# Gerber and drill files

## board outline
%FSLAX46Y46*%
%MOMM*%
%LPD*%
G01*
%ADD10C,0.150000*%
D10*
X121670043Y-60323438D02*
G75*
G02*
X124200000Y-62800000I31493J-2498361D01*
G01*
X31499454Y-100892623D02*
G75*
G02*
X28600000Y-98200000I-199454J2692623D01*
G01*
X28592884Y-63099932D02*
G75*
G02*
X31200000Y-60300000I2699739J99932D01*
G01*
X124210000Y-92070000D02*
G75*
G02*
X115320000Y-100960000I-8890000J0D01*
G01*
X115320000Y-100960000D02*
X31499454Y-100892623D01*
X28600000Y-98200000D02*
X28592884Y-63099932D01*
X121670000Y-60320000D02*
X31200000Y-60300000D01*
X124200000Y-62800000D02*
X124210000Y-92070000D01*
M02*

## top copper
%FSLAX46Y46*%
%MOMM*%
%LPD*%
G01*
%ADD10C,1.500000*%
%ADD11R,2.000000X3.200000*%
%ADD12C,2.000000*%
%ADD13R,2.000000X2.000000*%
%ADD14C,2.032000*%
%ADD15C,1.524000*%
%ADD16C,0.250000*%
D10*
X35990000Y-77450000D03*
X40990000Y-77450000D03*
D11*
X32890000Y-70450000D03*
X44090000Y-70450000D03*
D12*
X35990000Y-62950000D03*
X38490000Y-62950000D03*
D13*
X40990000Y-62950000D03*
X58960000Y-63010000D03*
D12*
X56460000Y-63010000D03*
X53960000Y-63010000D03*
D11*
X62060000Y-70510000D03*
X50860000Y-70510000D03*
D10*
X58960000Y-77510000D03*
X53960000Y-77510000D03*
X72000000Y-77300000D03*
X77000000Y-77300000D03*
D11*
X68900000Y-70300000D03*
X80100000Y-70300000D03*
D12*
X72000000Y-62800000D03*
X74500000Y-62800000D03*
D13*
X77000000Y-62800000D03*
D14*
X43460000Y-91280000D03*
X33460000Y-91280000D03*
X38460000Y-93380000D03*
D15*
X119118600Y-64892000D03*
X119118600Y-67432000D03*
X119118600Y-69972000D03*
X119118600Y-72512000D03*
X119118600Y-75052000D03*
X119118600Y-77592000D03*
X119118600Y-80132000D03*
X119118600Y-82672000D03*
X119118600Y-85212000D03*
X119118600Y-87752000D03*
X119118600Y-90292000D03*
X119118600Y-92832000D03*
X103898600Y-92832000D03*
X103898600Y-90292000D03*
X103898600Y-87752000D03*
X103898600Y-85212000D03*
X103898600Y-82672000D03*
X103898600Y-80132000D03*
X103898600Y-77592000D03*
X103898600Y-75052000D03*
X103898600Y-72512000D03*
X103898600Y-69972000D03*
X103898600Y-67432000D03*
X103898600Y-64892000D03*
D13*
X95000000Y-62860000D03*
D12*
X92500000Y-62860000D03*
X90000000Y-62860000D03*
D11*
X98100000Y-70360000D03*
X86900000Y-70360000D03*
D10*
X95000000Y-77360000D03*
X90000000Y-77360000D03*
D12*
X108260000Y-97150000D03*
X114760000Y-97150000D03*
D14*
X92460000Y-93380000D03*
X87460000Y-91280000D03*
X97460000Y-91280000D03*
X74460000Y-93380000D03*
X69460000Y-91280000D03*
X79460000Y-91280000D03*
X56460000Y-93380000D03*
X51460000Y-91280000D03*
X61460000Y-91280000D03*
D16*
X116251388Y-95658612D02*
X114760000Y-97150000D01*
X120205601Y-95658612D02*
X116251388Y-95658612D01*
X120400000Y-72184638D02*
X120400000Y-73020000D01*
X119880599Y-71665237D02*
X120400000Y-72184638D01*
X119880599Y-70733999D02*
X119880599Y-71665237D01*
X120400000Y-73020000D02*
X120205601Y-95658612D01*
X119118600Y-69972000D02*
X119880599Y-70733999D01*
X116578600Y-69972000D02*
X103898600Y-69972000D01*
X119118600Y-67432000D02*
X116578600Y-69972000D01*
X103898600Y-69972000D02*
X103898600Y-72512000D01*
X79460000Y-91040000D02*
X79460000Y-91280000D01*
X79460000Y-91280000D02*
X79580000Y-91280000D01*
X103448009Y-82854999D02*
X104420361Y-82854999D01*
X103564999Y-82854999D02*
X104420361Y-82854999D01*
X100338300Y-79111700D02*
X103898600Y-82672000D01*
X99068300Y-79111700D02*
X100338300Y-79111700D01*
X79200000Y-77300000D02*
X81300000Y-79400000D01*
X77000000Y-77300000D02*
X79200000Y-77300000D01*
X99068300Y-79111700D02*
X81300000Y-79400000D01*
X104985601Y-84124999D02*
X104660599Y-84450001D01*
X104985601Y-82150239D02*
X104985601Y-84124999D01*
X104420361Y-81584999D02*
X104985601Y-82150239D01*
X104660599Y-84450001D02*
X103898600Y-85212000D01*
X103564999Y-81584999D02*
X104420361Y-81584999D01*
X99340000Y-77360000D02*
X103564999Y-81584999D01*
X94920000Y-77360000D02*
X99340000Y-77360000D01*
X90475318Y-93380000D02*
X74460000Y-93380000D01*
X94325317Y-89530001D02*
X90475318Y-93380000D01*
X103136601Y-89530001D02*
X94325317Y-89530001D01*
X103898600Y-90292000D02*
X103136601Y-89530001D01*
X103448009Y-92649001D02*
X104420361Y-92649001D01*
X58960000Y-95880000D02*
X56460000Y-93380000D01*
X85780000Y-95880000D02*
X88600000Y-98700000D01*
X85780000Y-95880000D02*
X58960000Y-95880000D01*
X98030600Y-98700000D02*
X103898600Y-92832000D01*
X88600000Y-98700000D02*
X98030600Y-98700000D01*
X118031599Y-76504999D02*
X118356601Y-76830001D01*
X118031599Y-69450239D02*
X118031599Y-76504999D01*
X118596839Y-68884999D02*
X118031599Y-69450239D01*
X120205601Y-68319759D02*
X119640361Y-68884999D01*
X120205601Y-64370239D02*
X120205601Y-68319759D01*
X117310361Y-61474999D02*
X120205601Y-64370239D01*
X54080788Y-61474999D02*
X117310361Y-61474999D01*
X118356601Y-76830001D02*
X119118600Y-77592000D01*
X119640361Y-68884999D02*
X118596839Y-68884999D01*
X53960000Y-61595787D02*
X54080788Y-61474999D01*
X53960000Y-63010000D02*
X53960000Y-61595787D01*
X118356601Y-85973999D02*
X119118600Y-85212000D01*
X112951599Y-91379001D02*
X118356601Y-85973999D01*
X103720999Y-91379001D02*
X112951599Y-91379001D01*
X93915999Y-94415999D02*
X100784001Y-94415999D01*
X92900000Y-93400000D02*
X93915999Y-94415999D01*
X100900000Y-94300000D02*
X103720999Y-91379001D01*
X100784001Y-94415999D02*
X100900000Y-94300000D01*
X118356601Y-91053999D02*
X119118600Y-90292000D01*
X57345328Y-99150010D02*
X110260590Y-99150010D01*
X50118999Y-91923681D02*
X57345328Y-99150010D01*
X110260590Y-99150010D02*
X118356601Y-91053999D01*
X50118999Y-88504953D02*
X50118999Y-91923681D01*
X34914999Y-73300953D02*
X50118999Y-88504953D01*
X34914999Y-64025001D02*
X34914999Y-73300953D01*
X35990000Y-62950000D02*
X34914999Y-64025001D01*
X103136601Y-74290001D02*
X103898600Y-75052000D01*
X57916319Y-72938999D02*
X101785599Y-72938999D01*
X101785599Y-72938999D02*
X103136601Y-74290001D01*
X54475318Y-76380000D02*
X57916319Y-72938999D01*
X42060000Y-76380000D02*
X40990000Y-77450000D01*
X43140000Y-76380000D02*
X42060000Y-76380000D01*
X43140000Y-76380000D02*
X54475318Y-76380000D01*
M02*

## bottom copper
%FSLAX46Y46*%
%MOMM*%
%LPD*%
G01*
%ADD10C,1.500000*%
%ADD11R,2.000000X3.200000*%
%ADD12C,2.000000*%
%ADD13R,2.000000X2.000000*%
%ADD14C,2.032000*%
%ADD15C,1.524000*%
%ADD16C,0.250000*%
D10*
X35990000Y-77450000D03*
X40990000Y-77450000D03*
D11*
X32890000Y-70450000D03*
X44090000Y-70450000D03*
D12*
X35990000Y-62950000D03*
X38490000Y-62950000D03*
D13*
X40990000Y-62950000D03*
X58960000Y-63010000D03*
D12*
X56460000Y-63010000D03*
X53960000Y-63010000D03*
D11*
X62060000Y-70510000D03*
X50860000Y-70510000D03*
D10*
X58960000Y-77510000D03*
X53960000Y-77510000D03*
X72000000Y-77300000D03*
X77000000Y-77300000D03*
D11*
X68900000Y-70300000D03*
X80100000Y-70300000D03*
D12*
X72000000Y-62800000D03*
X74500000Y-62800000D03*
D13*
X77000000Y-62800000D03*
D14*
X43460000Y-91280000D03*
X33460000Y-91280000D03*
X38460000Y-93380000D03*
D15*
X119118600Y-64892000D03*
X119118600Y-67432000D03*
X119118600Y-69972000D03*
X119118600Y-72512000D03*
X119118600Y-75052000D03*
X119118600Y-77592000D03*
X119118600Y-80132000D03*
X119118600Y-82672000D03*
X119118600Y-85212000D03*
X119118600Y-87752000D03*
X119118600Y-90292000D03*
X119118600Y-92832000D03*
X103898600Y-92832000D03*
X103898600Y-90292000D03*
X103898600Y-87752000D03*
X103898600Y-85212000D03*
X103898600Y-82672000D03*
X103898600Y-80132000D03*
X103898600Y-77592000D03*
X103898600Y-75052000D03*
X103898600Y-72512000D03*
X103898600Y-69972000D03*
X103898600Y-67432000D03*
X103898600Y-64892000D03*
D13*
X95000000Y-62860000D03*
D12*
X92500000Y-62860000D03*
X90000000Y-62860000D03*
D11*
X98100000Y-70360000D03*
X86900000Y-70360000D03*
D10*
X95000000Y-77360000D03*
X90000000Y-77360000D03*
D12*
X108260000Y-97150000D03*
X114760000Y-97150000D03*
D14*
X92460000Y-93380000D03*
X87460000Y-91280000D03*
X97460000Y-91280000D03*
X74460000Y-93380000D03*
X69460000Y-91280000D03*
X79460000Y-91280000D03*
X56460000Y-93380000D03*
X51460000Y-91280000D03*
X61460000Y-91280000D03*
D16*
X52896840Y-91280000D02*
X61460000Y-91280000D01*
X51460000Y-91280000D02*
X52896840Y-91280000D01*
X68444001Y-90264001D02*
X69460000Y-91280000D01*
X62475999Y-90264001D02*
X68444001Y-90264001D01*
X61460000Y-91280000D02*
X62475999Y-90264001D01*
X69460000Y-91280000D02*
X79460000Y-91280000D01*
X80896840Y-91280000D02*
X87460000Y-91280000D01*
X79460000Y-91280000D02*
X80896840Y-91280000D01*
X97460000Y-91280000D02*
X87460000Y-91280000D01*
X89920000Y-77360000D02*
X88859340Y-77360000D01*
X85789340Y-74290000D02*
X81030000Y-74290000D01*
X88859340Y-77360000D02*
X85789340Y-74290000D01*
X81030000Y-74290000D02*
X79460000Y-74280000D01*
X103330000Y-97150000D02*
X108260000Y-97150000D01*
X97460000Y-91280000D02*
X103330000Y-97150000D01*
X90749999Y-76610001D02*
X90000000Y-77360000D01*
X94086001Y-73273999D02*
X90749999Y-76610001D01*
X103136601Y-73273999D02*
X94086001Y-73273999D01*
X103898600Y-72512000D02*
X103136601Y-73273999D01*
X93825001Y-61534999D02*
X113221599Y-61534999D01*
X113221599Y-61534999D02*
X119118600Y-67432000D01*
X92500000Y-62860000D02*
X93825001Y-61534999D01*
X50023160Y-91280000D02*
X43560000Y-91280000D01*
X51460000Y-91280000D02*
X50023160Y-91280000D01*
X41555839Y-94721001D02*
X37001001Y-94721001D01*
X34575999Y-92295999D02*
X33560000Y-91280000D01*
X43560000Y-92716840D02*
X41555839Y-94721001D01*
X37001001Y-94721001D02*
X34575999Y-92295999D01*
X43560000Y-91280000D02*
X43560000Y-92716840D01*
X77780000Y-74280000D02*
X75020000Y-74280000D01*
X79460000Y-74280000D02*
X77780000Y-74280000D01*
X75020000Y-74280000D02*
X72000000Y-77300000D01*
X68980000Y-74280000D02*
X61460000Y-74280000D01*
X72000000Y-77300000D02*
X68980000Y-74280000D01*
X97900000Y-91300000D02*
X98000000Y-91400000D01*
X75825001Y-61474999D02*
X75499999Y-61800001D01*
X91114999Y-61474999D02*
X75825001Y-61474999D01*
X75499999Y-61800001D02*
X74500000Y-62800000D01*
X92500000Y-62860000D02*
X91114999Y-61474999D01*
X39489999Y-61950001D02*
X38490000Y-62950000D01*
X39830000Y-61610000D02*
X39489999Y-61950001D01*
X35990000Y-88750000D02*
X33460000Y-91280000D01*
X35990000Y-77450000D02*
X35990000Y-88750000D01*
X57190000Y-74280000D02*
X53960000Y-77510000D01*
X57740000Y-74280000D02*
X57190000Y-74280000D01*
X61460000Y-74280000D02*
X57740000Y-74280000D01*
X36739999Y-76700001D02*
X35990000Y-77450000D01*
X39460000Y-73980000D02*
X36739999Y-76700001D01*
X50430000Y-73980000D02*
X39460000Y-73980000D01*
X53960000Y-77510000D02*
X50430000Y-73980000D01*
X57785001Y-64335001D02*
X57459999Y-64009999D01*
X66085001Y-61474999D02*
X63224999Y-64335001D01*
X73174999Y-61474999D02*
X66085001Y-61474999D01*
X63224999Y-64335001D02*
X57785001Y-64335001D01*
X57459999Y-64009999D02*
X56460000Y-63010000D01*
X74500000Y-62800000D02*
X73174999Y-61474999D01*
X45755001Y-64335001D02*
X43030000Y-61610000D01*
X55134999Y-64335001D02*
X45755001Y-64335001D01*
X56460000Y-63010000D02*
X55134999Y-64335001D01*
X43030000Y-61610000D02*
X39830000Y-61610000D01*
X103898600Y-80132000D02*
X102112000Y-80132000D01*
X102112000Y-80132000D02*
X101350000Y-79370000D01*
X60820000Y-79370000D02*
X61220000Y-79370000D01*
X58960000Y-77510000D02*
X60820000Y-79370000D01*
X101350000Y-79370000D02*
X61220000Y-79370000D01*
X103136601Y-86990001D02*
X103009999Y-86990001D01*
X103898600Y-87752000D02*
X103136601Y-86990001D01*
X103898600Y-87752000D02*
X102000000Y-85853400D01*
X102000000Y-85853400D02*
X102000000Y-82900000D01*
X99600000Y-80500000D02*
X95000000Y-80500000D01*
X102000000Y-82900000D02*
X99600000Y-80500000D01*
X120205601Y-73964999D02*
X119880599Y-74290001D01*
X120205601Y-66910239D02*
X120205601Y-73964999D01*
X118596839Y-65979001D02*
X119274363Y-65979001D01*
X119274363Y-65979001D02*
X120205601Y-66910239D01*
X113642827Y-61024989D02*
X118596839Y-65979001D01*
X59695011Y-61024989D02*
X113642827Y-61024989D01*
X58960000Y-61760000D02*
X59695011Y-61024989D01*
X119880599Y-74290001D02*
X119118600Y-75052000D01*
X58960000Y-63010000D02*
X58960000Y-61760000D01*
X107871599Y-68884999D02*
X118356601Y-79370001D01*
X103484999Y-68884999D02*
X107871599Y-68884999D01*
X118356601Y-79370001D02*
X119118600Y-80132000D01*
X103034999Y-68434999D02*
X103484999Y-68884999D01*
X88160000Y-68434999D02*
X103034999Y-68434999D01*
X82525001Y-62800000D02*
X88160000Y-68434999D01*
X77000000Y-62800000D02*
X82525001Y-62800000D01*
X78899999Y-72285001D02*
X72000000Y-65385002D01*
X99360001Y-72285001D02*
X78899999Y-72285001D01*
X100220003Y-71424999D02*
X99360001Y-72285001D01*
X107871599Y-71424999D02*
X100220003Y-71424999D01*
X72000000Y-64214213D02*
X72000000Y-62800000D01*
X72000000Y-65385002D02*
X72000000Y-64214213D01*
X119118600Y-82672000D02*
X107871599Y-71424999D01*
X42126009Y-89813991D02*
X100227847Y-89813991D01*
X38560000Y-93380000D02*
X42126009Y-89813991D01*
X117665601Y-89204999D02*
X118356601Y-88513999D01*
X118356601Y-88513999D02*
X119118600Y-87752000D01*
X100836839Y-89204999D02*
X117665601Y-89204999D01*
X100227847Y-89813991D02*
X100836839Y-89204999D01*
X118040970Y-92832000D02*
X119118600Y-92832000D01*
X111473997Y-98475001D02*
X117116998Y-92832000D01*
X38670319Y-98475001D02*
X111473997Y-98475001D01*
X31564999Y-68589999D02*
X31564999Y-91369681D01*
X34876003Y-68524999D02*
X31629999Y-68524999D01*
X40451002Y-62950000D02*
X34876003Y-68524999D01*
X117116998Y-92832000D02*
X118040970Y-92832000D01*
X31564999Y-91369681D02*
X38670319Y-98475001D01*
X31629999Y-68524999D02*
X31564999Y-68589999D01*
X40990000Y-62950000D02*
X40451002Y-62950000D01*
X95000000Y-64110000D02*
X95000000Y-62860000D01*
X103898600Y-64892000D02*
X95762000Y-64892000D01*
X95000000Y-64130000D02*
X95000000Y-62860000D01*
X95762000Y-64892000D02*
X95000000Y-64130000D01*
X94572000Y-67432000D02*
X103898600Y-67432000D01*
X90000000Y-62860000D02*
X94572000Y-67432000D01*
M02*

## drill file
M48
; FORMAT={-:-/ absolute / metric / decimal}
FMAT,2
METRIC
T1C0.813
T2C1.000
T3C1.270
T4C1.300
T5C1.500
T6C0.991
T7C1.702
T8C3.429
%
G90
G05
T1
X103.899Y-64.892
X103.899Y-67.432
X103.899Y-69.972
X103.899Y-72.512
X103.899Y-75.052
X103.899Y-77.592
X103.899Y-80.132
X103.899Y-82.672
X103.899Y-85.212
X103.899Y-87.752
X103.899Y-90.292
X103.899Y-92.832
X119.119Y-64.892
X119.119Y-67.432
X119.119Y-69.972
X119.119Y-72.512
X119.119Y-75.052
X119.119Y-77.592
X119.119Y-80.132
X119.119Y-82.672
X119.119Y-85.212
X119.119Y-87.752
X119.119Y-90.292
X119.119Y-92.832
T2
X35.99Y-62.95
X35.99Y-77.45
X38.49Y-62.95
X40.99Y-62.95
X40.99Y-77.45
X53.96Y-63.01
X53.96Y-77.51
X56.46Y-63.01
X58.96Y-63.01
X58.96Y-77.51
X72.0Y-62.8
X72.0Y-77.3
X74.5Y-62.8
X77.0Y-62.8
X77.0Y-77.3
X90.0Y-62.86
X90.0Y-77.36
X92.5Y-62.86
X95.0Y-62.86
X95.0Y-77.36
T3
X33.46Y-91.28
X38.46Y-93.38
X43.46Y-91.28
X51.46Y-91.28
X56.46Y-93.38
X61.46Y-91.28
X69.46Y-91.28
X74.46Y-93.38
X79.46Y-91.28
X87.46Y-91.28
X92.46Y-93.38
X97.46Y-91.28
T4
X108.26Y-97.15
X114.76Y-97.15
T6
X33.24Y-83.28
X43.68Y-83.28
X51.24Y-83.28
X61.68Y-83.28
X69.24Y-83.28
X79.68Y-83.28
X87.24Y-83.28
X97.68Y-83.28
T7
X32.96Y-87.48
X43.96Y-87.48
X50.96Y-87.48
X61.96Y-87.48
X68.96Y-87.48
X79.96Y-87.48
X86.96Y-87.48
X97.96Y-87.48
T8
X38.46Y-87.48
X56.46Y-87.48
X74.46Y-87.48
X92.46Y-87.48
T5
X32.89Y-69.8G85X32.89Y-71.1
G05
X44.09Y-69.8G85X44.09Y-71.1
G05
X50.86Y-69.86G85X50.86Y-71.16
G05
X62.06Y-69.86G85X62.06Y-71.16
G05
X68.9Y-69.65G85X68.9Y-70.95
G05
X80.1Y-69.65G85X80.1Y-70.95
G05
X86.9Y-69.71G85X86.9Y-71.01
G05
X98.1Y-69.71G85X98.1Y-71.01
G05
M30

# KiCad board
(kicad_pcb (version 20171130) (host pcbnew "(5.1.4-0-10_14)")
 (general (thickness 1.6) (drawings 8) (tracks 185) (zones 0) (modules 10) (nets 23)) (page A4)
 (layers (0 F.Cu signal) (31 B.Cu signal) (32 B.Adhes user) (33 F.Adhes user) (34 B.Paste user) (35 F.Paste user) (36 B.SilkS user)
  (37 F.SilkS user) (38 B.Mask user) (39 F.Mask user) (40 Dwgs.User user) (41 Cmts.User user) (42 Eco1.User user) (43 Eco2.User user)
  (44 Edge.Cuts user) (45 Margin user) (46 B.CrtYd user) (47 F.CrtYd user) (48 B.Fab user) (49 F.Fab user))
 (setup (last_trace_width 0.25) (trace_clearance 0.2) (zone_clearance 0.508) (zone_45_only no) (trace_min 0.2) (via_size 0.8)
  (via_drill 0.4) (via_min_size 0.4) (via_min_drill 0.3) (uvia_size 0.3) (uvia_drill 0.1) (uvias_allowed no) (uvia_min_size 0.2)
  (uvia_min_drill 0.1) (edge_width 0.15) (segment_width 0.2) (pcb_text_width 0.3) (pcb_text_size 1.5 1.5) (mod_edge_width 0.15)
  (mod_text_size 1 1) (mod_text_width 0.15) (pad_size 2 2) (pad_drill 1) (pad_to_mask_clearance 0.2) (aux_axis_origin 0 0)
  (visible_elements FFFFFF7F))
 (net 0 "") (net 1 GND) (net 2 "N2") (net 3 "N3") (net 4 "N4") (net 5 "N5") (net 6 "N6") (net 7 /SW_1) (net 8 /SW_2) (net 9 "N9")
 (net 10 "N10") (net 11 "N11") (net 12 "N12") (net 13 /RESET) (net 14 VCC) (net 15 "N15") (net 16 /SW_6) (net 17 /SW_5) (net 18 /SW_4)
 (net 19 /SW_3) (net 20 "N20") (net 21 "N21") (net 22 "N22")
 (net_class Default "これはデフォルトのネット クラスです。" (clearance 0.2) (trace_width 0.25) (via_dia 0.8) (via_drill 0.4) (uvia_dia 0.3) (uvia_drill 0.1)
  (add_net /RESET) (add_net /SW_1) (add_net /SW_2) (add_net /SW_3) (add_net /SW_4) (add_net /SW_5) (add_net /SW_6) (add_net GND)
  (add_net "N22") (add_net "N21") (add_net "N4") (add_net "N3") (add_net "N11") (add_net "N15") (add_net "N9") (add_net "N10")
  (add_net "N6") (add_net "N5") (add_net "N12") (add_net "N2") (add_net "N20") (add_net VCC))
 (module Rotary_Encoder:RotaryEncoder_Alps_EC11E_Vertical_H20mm (layer F.Cu) (at 40.99 62.95 270)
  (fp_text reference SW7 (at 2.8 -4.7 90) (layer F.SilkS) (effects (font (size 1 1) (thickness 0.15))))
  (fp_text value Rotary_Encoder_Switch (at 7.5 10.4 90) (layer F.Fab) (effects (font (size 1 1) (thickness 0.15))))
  (pad "" thru_hole circle (at 14.5 5 270) (size 1.5 1.5) (drill 1) (layers *.Cu *.Mask) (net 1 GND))
  (pad "" thru_hole circle (at 14.5 0 270) (size 1.5 1.5) (drill 1) (layers *.Cu *.Mask) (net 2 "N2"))
  (pad MP thru_hole rect (at 7.5 8.1 270) (size 3.2 2) (drill oval 2.8 1.5) (layers *.Cu *.Mask))
  (pad MP thru_hole rect (at 7.5 -3.1 270) (size 3.2 2) (drill oval 2.8 1.5) (layers *.Cu *.Mask))
  (pad B thru_hole circle (at 0 5 270) (size 2 2) (drill 1) (layers *.Cu *.Mask) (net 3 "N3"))
  (pad C thru_hole circle (at 0 2.5 270) (size 2 2) (drill 1) (layers *.Cu *.Mask) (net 1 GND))
  (pad A thru_hole rect (at 0 0 270) (size 2 2) (drill 1) (layers *.Cu *.Mask) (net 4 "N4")))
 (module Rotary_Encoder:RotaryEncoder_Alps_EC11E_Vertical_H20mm (layer F.Cu) (at 58.96 63.01 270)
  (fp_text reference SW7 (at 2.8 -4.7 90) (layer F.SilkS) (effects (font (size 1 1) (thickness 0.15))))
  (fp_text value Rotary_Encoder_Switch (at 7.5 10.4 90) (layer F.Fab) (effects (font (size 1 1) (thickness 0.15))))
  (pad A thru_hole rect (at 0 0 270) (size 2 2) (drill 1) (layers *.Cu *.Mask) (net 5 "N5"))
  (pad C thru_hole circle (at 0 2.5 270) (size 2 2) (drill 1) (layers *.Cu *.Mask) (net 1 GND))
  (pad B thru_hole circle (at 0 5 270) (size 2 2) (drill 1) (layers *.Cu *.Mask) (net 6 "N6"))
  (pad MP thru_hole rect (at 7.5 -3.1 270) (size 3.2 2) (drill oval 2.8 1.5) (layers *.Cu *.Mask))
  (pad MP thru_hole rect (at 7.5 8.1 270) (size 3.2 2) (drill oval 2.8 1.5) (layers *.Cu *.Mask))
  (pad "" thru_hole circle (at 14.5 0 270) (size 1.5 1.5) (drill 1) (layers *.Cu *.Mask) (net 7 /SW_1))
  (pad "" thru_hole circle (at 14.5 5 270) (size 1.5 1.5) (drill 1) (layers *.Cu *.Mask) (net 1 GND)))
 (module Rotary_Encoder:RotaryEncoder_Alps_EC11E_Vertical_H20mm (layer F.Cu) (at 77 62.8 270)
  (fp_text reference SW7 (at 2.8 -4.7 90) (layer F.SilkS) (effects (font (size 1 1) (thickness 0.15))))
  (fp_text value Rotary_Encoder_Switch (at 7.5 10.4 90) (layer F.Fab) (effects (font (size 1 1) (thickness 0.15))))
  (pad "" thru_hole circle (at 14.5 5 270) (size 1.5 1.5) (drill 1) (layers *.Cu *.Mask) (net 1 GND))
  (pad "" thru_hole circle (at 14.5 0 270) (size 1.5 1.5) (drill 1) (layers *.Cu *.Mask) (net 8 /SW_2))
  (pad MP thru_hole rect (at 7.5 8.1 270) (size 3.2 2) (drill oval 2.8 1.5) (layers *.Cu *.Mask))
  (pad MP thru_hole rect (at 7.5 -3.1 270) (size 3.2 2) (drill oval 2.8 1.5) (layers *.Cu *.Mask))
  (pad B thru_hole circle (at 0 5 270) (size 2 2) (drill 1) (layers *.Cu *.Mask) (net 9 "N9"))
  (pad C thru_hole circle (at 0 2.5 270) (size 2 2) (drill 1) (layers *.Cu *.Mask) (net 1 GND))
  (pad A thru_hole rect (at 0 0 270) (size 2 2) (drill 1) (layers *.Cu *.Mask) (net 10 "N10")))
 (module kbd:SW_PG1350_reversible (layer F.Cu) (at 38.46 87.48)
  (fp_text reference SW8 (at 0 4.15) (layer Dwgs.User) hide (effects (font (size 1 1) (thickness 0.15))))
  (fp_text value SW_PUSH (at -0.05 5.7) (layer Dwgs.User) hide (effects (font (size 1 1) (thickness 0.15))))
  (pad "" np_thru_hole circle (at -5.22 -4.2) (size 0.9906 0.9906) (drill 0.9906) (layers *.Cu *.Mask))
  (pad 2 thru_hole circle (at 5 3.8) (size 2.032 2.032) (drill 1.27) (layers *.Cu *.Mask) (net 1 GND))
  (pad "" np_thru_hole circle (at 0 0) (size 3.429 3.429) (drill 3.429) (layers *.Cu *.Mask))
  (pad 2 thru_hole circle (at -5 3.8) (size 2.032 2.032) (drill 1.27) (layers *.Cu *.Mask) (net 1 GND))
  (pad 1 thru_hole circle (at 0 5.9) (size 2.032 2.032) (drill 1.27) (layers *.Cu *.Mask) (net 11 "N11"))
  (pad "" np_thru_hole circle (at 5.22 -4.2) (size 0.9906 0.9906) (drill 0.9906) (layers *.Cu *.Mask))
  (pad "" np_thru_hole circle (at 5.5 0) (size 1.7018 1.7018) (drill 1.7018) (layers *.Cu *.Mask))
  (pad "" np_thru_hole circle (at -5.5 0) (size 1.7018 1.7018) (drill 1.7018) (layers *.Cu *.Mask)))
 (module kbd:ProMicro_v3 (layer B.Cu) (at 111.51 79.37 180)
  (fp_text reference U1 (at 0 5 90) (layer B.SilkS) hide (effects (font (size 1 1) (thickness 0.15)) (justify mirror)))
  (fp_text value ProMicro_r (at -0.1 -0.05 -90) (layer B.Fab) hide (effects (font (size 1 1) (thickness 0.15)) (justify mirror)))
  (pad 24 thru_hole circle (at -7.6086 14.478 180) (size 1.524 1.524) (drill 0.8128) (layers *.Cu *.Mask B.SilkS) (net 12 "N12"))
  (pad 23 thru_hole circle (at -7.6086 11.938 180) (size 1.524 1.524) (drill 0.8128) (layers *.Cu *.Mask B.SilkS) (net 1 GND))
  (pad 22 thru_hole circle (at -7.6086 9.398 180) (size 1.524 1.524) (drill 0.8128) (layers *.Cu *.Mask B.SilkS) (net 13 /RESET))
  (pad 21 thru_hole circle (at -7.6086 6.858 180) (size 1.524 1.524) (drill 0.8128) (layers *.Cu *.Mask B.SilkS) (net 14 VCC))
  (pad 20 thru_hole circle (at -7.6086 4.318 180) (size 1.524 1.524) (drill 0.8128) (layers *.Cu *.Mask B.SilkS) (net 5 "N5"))
  (pad 19 thru_hole circle (at -7.6086 1.778 180) (size 1.524 1.524) (drill 0.8128) (layers *.Cu *.Mask B.SilkS) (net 6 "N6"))
  (pad 18 thru_hole circle (at -7.6086 -0.762 180) (size 1.524 1.524) (drill 0.8128) (layers *.Cu *.Mask B.SilkS) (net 10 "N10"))
  (pad 17 thru_hole circle (at -7.6086 -3.302 180) (size 1.524 1.524) (drill 0.8128) (layers *.Cu *.Mask B.SilkS) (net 9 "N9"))
  (pad 16 thru_hole circle (at -7.6086 -5.842 180) (size 1.524 1.524) (drill 0.8128) (layers *.Cu *.Mask B.SilkS) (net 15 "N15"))
  (pad 15 thru_hole circle (at -7.6086 -8.382 180) (size 1.524 1.524) (drill 0.8128) (layers *.Cu *.Mask B.SilkS) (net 11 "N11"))
  (pad 14 thru_hole circle (at -7.6086 -10.922 180) (size 1.524 1.524) (drill 0.8128) (layers *.Cu *.Mask B.SilkS) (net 3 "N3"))
  (pad 13 thru_hole circle (at -7.6086 -13.462 180) (size 1.524 1.524) (drill 0.8128) (layers *.Cu *.Mask B.SilkS) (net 4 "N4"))
  (pad 12 thru_hole circle (at 7.6114 -13.462 180) (size 1.524 1.524) (drill 0.8128) (layers *.Cu *.Mask B.SilkS) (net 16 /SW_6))
  (pad 11 thru_hole circle (at 7.6114 -10.922 180) (size 1.524 1.524) (drill 0.8128) (layers *.Cu *.Mask B.SilkS) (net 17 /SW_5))
  (pad 10 thru_hole circle (at 7.6114 -8.382 180) (size 1.524 1.524) (drill 0.8128) (layers *.Cu *.Mask B.SilkS) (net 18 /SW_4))
  (pad 9 thru_hole circle (at 7.6114 -5.842 180) (size 1.524 1.524) (drill 0.8128) (layers *.Cu *.Mask B.SilkS) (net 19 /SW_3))
  (pad 8 thru_hole circle (at 7.6114 -3.302 180) (size 1.524 1.524) (drill 0.8128) (layers *.Cu *.Mask B.SilkS) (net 8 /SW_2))
  (pad 7 thru_hole circle (at 7.6114 -0.762 180) (size 1.524 1.524) (drill 0.8128) (layers *.Cu *.Mask B.SilkS) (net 7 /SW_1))
  (pad 6 thru_hole circle (at 7.6114 1.778 180) (size 1.524 1.524) (drill 0.8128) (layers *.Cu *.Mask B.SilkS) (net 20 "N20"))
  (pad 5 thru_hole circle (at 7.6114 4.318 180) (size 1.524 1.524) (drill 0.8128) (layers *.Cu *.Mask B.SilkS) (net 2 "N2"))
  (pad 4 thru_hole circle (at 7.6114 6.858 180) (size 1.524 1.524) (drill 0.8128) (layers *.Cu *.Mask B.SilkS) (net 1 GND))
  (pad 3 thru_hole circle (at 7.6114 9.398 180) (size 1.524 1.524) (drill 0.8128) (layers *.Cu *.Mask B.SilkS) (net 1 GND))
  (pad 2 thru_hole circle (at 7.6114 11.938 180) (size 1.524 1.524) (drill 0.8128) (layers *.Cu *.Mask B.SilkS) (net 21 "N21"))
  (pad 1 thru_hole circle (at 7.6114 14.478 180) (size 1.524 1.524) (drill 0.8128) (layers *.Cu *.Mask B.SilkS) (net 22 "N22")))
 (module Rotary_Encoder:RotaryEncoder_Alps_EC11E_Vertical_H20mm (layer F.Cu) (at 95 62.86 270)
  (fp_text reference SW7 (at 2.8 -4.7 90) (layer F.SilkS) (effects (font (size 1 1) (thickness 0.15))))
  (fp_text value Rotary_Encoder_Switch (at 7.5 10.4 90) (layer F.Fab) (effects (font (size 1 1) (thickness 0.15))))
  (pad A thru_hole rect (at 0 0 270) (size 2 2) (drill 1) (layers *.Cu *.Mask) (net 22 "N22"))
  (pad C thru_hole circle (at 0 2.5 270) (size 2 2) (drill 1) (layers *.Cu *.Mask) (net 1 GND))
  (pad B thru_hole circle (at 0 5 270) (size 2 2) (drill 1) (layers *.Cu *.Mask) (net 21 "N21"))
  (pad MP thru_hole rect (at 7.5 -3.1 270) (size 3.2 2) (drill oval 2.8 1.5) (layers *.Cu *.Mask))
  (pad MP thru_hole rect (at 7.5 8.1 270) (size 3.2 2) (drill oval 2.8 1.5) (layers *.Cu *.Mask))
  (pad "" thru_hole circle (at 14.5 0 270) (size 1.5 1.5) (drill 1) (layers *.Cu *.Mask) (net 19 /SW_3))
  (pad "" thru_hole circle (at 14.5 5 270) (size 1.5 1.5) (drill 1) (layers *.Cu *.Mask) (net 1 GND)))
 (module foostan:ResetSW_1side (layer F.Cu) (at 111.51 97.15)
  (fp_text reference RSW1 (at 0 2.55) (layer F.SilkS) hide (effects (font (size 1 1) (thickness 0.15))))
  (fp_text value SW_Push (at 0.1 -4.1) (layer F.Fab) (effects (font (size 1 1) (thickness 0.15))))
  (pad 2 thru_hole circle (at -3.25 0) (size 2 2) (drill 1.3) (layers *.Cu F.SilkS B.Mask) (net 1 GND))
  (pad 1 thru_hole circle (at 3.25 0) (size 2 2) (drill 1.3) (layers *.Cu F.SilkS B.Mask) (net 13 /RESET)))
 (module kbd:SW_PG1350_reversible (layer F.Cu) (at 92.46 87.48)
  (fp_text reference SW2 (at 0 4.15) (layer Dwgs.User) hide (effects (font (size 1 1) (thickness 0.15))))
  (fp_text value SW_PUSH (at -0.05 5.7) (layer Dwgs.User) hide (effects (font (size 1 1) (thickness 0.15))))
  (pad "" np_thru_hole circle (at -5.5 0) (size 1.7018 1.7018) (drill 1.7018) (layers *.Cu *.Mask))
  (pad "" np_thru_hole circle (at 5.5 0) (size 1.7018 1.7018) (drill 1.7018) (layers *.Cu *.Mask))
  (pad "" np_thru_hole circle (at 5.22 -4.2) (size 0.9906 0.9906) (drill 0.9906) (layers *.Cu *.Mask))
  (pad 1 thru_hole circle (at 0 5.9) (size 2.032 2.032) (drill 1.27) (layers *.Cu *.Mask) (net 15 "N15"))
  (pad 2 thru_hole circle (at -5 3.8) (size 2.032 2.032) (drill 1.27) (layers *.Cu *.Mask) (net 1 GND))
  (pad "" np_thru_hole circle (at 0 0) (size 3.429 3.429) (drill 3.429) (layers *.Cu *.Mask))
  (pad 2 thru_hole circle (at 5 3.8) (size 2.032 2.032) (drill 1.27) (layers *.Cu *.Mask) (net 1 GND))
  (pad "" np_thru_hole circle (at -5.22 -4.2) (size 0.9906 0.9906) (drill 0.9906) (layers *.Cu *.Mask)))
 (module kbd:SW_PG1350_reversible (layer F.Cu) (at 74.46 87.48)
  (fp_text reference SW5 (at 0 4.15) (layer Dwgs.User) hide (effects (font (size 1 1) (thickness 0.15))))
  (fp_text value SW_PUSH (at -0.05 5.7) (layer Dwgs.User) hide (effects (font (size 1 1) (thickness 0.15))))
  (pad "" np_thru_hole circle (at -5.5 0) (size 1.7018 1.7018) (drill 1.7018) (layers *.Cu *.Mask))
  (pad "" np_thru_hole circle (at 5.5 0) (size 1.7018 1.7018) (drill 1.7018) (layers *.Cu *.Mask))
  (pad "" np_thru_hole circle (at 5.22 -4.2) (size 0.9906 0.9906) (drill 0.9906) (layers *.Cu *.Mask))
  (pad 1 thru_hole circle (at 0 5.9) (size 2.032 2.032) (drill 1.27) (layers *.Cu *.Mask) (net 17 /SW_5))
  (pad 2 thru_hole circle (at -5 3.8) (size 2.032 2.032) (drill 1.27) (layers *.Cu *.Mask) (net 1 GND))
  (pad "" np_thru_hole circle (at 0 0) (size 3.429 3.429) (drill 3.429) (layers *.Cu *.Mask))
  (pad 2 thru_hole circle (at 5 3.8) (size 2.032 2.032) (drill 1.27) (layers *.Cu *.Mask) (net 1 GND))
  (pad "" np_thru_hole circle (at -5.22 -4.2) (size 0.9906 0.9906) (drill 0.9906) (layers *.Cu *.Mask)))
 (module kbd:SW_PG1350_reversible (layer F.Cu) (at 56.46 87.48)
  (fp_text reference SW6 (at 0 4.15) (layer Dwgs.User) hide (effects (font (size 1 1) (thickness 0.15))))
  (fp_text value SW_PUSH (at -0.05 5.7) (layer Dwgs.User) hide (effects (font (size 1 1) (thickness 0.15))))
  (pad "" np_thru_hole circle (at -5.5 0) (size 1.7018 1.7018) (drill 1.7018) (layers *.Cu *.Mask))
  (pad "" np_thru_hole circle (at 5.5 0) (size 1.7018 1.7018) (drill 1.7018) (layers *.Cu *.Mask))
  (pad "" np_thru_hole circle (at 5.22 -4.2) (size 0.9906 0.9906) (drill 0.9906) (layers *.Cu *.Mask))
  (pad 1 thru_hole circle (at 0 5.9) (size 2.032 2.032) (drill 1.27) (layers *.Cu *.Mask) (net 16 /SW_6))
  (pad 2 thru_hole circle (at -5 3.8) (size 2.032 2.032) (drill 1.27) (layers *.Cu *.Mask) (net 1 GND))
  (pad "" np_thru_hole circle (at 0 0) (size 3.429 3.429) (drill 3.429) (layers *.Cu *.Mask))
  (pad 2 thru_hole circle (at 5 3.8) (size 2.032 2.032) (drill 1.27) (layers *.Cu *.Mask) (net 1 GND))
  (pad "" np_thru_hole circle (at -5.22 -4.2) (size 0.9906 0.9906) (drill 0.9906) (layers *.Cu *.Mask)))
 (gr_arc (start 121.701536 62.821799) (end 124.2 62.8) (angle -90.22231091) (layer Edge.Cuts) (width 0.15))
 (gr_arc (start 31.3 98.2) (end 28.6 98.2) (angle -94.2363948) (layer Edge.Cuts) (width 0.15))
 (gr_arc (start 31.292623 63) (end 31.2 60.3) (angle -90.15510012) (layer Edge.Cuts) (width 0.15))
 (gr_arc (start 115.32 92.07) (end 115.32 100.96) (angle -90) (layer Edge.Cuts) (width 0.15))
 (gr_line (start 115.32 100.96) (end 31.499454 100.892623) (layer Edge.Cuts) (width 0.15))
 (gr_line (start 28.6 98.2) (end 28.592884 63.099932) (layer Edge.Cuts) (width 0.15))
 (gr_line (start 121.67 60.32) (end 31.2 60.3) (layer Edge.Cuts) (width 0.15))
 (gr_line (start 124.2 62.8) (end 124.21 92.07) (layer Edge.Cuts) (width 0.15))
 (segment (start 116.251388 95.658612) (end 114.76 97.15) (width 0.25) (layer F.Cu) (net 13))
 (segment (start 120.205601 95.658612) (end 116.251388 95.658612) (width 0.25) (layer F.Cu) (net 13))
 (segment (start 120.4 72.184638) (end 120.4 73.02) (width 0.25) (layer F.Cu) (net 13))
 (segment (start 119.880599 71.665237) (end 120.4 72.184638) (width 0.25) (layer F.Cu) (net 13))
 (segment (start 119.880599 70.733999) (end 119.880599 71.665237) (width 0.25) (layer F.Cu) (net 13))
 (segment (start 120.4 73.02) (end 120.205601 95.658612) (width 0.25) (layer F.Cu) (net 13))
 (segment (start 119.1186 69.972) (end 119.880599 70.733999) (width 0.25) (layer F.Cu) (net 13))
 (segment (start 52.89684 91.28) (end 61.46 91.28) (width 0.25) (layer B.Cu) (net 1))
 (segment (start 51.46 91.28) (end 52.89684 91.28) (width 0.25) (layer B.Cu) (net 1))
 (segment (start 68.444001 90.264001) (end 69.46 91.28) (width 0.25) (layer B.Cu) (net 1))
 (segment (start 62.475999 90.264001) (end 68.444001 90.264001) (width 0.25) (layer B.Cu) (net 1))
 (segment (start 61.46 91.28) (end 62.475999 90.264001) (width 0.25) (layer B.Cu) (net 1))
 (segment (start 69.46 91.28) (end 79.46 91.28) (width 0.25) (layer B.Cu) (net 1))
 (segment (start 80.89684 91.28) (end 87.46 91.28) (width 0.25) (layer B.Cu) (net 1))
 (segment (start 79.46 91.28) (end 80.89684 91.28) (width 0.25) (layer B.Cu) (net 1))
 (segment (start 97.46 91.28) (end 87.46 91.28) (width 0.25) (layer B.Cu) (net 1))
 (segment (start 89.92 77.36) (end 88.85934 77.36) (width 0.25) (layer B.Cu) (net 1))
 (segment (start 85.78934 74.29) (end 81.03 74.29) (width 0.25) (layer B.Cu) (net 1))
 (segment (start 88.85934 77.36) (end 85.78934 74.29) (width 0.25) (layer B.Cu) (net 1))
 (segment (start 81.03 74.29) (end 79.46 74.28) (width 0.25) (layer B.Cu) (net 1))
 (segment (start 103.33 97.15) (end 108.26 97.15) (width 0.25) (layer B.Cu) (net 1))
 (segment (start 97.46 91.28) (end 103.33 97.15) (width 0.25) (layer B.Cu) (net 1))
 (segment (start 90.749999 76.610001) (end 90 77.36) (width 0.25) (layer B.Cu) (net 1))
 (segment (start 94.086001 73.273999) (end 90.749999 76.610001) (width 0.25) (layer B.Cu) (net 1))
 (segment (start 103.136601 73.273999) (end 94.086001 73.273999) (width 0.25) (layer B.Cu) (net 1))
 (segment (start 103.8986 72.512) (end 103.136601 73.273999) (width 0.25) (layer B.Cu) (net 1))
 (segment (start 116.5786 69.972) (end 103.8986 69.972) (width 0.25) (layer F.Cu) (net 1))
 (segment (start 119.1186 67.432) (end 116.5786 69.972) (width 0.25) (layer F.Cu) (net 1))
 (segment (start 103.8986 69.972) (end 103.8986 72.512) (width 0.25) (layer F.Cu) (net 1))
 (segment (start 93.825001 61.534999) (end 113.221599 61.534999) (width 0.25) (layer B.Cu) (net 1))
 (segment (start 113.221599 61.534999) (end 119.1186 67.432) (width 0.25) (layer B.Cu) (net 1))
 (segment (start 92.5 62.86) (end 93.825001 61.534999) (width 0.25) (layer B.Cu) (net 1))
 (segment (start 50.02316 91.28) (end 43.56 91.28) (width 0.25) (layer B.Cu) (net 1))
 (segment (start 51.46 91.28) (end 50.02316 91.28) (width 0.25) (layer B.Cu) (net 1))
 (segment (start 41.555839 94.721001) (end 37.001001 94.721001) (width 0.25) (layer B.Cu) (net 1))
 (segment (start 34.575999 92.295999) (end 33.56 91.28) (width 0.25) (layer B.Cu) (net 1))
 (segment (start 43.56 92.71684) (end 41.555839 94.721001) (width 0.25) (layer B.Cu) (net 1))
 (segment (start 37.001001 94.721001) (end 34.575999 92.295999) (width 0.25) (layer B.Cu) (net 1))
 (segment (start 43.56 91.28) (end 43.56 92.71684) (width 0.25) (layer B.Cu) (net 1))
 (segment (start 79.46 91.04) (end 79.46 91.28) (width 0.25) (layer F.Cu) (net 1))
 (segment (start 79.46 91.28) (end 79.58 91.28) (width 0.25) (layer F.Cu) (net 1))
 (segment (start 77.78 74.28) (end 75.02 74.28) (width 0.25) (layer B.Cu) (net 1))
 (segment (start 79.46 74.28) (end 77.78 74.28) (width 0.25) (layer B.Cu) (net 1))
 (segment (start 75.02 74.28) (end 72 77.3) (width 0.25) (layer B.Cu) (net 1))
 (segment (start 68.98 74.28) (end 61.46 74.28) (width 0.25) (layer B.Cu) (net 1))
 (segment (start 72 77.3) (end 68.98 74.28) (width 0.25) (layer B.Cu) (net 1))
 (segment (start 97.9 91.3) (end 98 91.4) (width 0.25) (layer B.Cu) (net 1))
 (segment (start 75.825001 61.474999) (end 75.499999 61.800001) (width 0.25) (layer B.Cu) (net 1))
 (segment (start 91.114999 61.474999) (end 75.825001 61.474999) (width 0.25) (layer B.Cu) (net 1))
 (segment (start 75.499999 61.800001) (end 74.5 62.8) (width 0.25) (layer B.Cu) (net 1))
 (segment (start 92.5 62.86) (end 91.114999 61.474999) (width 0.25) (layer B.Cu) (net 1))
 (segment (start 39.489999 61.950001) (end 38.49 62.95) (width 0.25) (layer B.Cu) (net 1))
 (segment (start 39.83 61.61) (end 39.489999 61.950001) (width 0.25) (layer B.Cu) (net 1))
 (segment (start 35.99 88.75) (end 33.46 91.28) (width 0.25) (layer B.Cu) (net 1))
 (segment (start 35.99 77.45) (end 35.99 88.75) (width 0.25) (layer B.Cu) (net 1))
 (segment (start 57.19 74.28) (end 53.96 77.51) (width 0.25) (layer B.Cu) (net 1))
 (segment (start 57.74 74.28) (end 57.19 74.28) (width 0.25) (layer B.Cu) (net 1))
 (segment (start 61.46 74.28) (end 57.74 74.28) (width 0.25) (layer B.Cu) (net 1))
 (segment (start 36.739999 76.700001) (end 35.99 77.45) (width 0.25) (layer B.Cu) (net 1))
 (segment (start 39.46 73.98) (end 36.739999 76.700001) (width 0.25) (layer B.Cu) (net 1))
 (segment (start 50.43 73.98) (end 39.46 73.98) (width 0.25) (layer B.Cu) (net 1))
 (segment (start 53.96 77.51) (end 50.43 73.98) (width 0.25) (layer B.Cu) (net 1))
 (segment (start 57.785001 64.335001) (end 57.459999 64.009999) (width 0.25) (layer B.Cu) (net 1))
 (segment (start 66.085001 61.474999) (end 63.224999 64.335001) (width 0.25) (layer B.Cu) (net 1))
 (segment (start 73.174999 61.474999) (end 66.085001 61.474999) (width 0.25) (layer B.Cu) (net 1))
 (segment (start 63.224999 64.335001) (end 57.785001 64.335001) (width 0.25) (layer B.Cu) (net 1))
 (segment (start 57.459999 64.009999) (end 56.46 63.01) (width 0.25) (layer B.Cu) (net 1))
 (segment (start 74.5 62.8) (end 73.174999 61.474999) (width 0.25) (layer B.Cu) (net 1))
 (segment (start 45.755001 64.335001) (end 43.03 61.61) (width 0.25) (layer B.Cu) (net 1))
 (segment (start 55.134999 64.335001) (end 45.755001 64.335001) (width 0.25) (layer B.Cu) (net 1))
 (segment (start 56.46 63.01) (end 55.134999 64.335001) (width 0.25) (layer B.Cu) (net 1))
 (segment (start 43.03 61.61) (end 39.83 61.61) (width 0.25) (layer B.Cu) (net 1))
 (segment (start 103.8986 80.132) (end 102.112 80.132) (width 0.25) (layer B.Cu) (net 7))
 (segment (start 102.112 80.132) (end 101.35 79.37) (width 0.25) (layer B.Cu) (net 7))
 (segment (start 60.82 79.37) (end 61.22 79.37) (width 0.25) (layer B.Cu) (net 7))
 (segment (start 58.96 77.51) (end 60.82 79.37) (width 0.25) (layer B.Cu) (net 7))
 (segment (start 101.35 79.37) (end 61.22 79.37) (width 0.25) (layer B.Cu) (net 7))
 (segment (start 103.448009 82.854999) (end 104.420361 82.854999) (width 0.25) (layer F.Cu) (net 8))
 (segment (start 103.564999 82.854999) (end 104.420361 82.854999) (width 0.25) (layer F.Cu) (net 8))
 (segment (start 100.3383 79.1117) (end 103.8986 82.672) (width 0.25) (layer F.Cu) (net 8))
 (segment (start 99.0683 79.1117) (end 100.3383 79.1117) (width 0.25) (layer F.Cu) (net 8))
 (segment (start 79.2 77.3) (end 81.3 79.4) (width 0.25) (layer F.Cu) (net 8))
 (segment (start 77 77.3) (end 79.2 77.3) (width 0.25) (layer F.Cu) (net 8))
 (segment (start 99.0683 79.1117) (end 81.3 79.4) (width 0.25) (layer F.Cu) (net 8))
 (segment (start 104.985601 84.124999) (end 104.660599 84.450001) (width 0.25) (layer F.Cu) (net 19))
 (segment (start 104.985601 82.150239) (end 104.985601 84.124999) (width 0.25) (layer F.Cu) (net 19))
 (segment (start 104.420361 81.584999) (end 104.985601 82.150239) (width 0.25) (layer F.Cu) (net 19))
 (segment (start 104.660599 84.450001) (end 103.8986 85.212) (width 0.25) (layer F.Cu) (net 19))
 (segment (start 103.564999 81.584999) (end 104.420361 81.584999) (width 0.25) (layer F.Cu) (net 19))
 (segment (start 99.34 77.36) (end 103.564999 81.584999) (width 0.25) (layer F.Cu) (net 19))
 (segment (start 94.92 77.36) (end 99.34 77.36) (width 0.25) (layer F.Cu) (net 19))
 (segment (start 103.136601 86.990001) (end 103.009999 86.990001) (width 0.25) (layer B.Cu) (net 18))
 (segment (start 103.8986 87.752) (end 103.136601 86.990001) (width 0.25) (layer B.Cu) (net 18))
 (segment (start 103.8986 87.752) (end 102 85.8534) (width 0.25) (layer B.Cu) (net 18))
 (segment (start 102 85.8534) (end 102 82.9) (width 0.25) (layer B.Cu) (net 18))
 (segment (start 99.6 80.5) (end 95 80.5) (width 0.25) (layer B.Cu) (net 18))
 (segment (start 102 82.9) (end 99.6 80.5) (width 0.25) (layer B.Cu) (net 18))
 (segment (start 90.475318 93.38) (end 74.46 93.38) (width 0.25) (layer F.Cu) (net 17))
 (segment (start 94.325317 89.530001) (end 90.475318 93.38) (width 0.25) (layer F.Cu) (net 17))
 (segment (start 103.136601 89.530001) (end 94.325317 89.530001) (width 0.25) (layer F.Cu) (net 17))
 (segment (start 103.8986 90.292) (end 103.136601 89.530001) (width 0.25) (layer F.Cu) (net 17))
 (segment (start 103.448009 92.649001) (end 104.420361 92.649001) (width 0.25) (layer F.Cu) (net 16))
 (segment (start 58.96 95.88) (end 56.46 93.38) (width 0.25) (layer F.Cu) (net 16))
 (segment (start 85.78 95.88) (end 88.6 98.7) (width 0.25) (layer F.Cu) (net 16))
 (segment (start 85.78 95.88) (end 58.96 95.88) (width 0.25) (layer F.Cu) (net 16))
 (segment (start 98.0306 98.7) (end 103.8986 92.832) (width 0.25) (layer F.Cu) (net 16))
 (segment (start 88.6 98.7) (end 98.0306 98.7) (width 0.25) (layer F.Cu) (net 16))
 (segment (start 120.205601 73.964999) (end 119.880599 74.290001) (width 0.25) (layer B.Cu) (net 5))
 (segment (start 120.205601 66.910239) (end 120.205601 73.964999) (width 0.25) (layer B.Cu) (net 5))
 (segment (start 118.596839 65.979001) (end 119.274363 65.979001) (width 0.25) (layer B.Cu) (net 5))
 (segment (start 119.274363 65.979001) (end 120.205601 66.910239) (width 0.25) (layer B.Cu) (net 5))
 (segment (start 113.642827 61.024989) (end 118.596839 65.979001) (width 0.25) (layer B.Cu) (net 5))
 (segment (start 59.695011 61.024989) (end 113.642827 61.024989) (width 0.25) (layer B.Cu) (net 5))
 (segment (start 58.96 61.76) (end 59.695011 61.024989) (width 0.25) (layer B.Cu) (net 5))
 (segment (start 119.880599 74.290001) (end 119.1186 75.052) (width 0.25) (layer B.Cu) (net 5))
 (segment (start 58.96 63.01) (end 58.96 61.76) (width 0.25) (layer B.Cu) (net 5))
 (segment (start 118.031599 76.504999) (end 118.356601 76.830001) (width 0.25) (layer F.Cu) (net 6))
 (segment (start 118.031599 69.450239) (end 118.031599 76.504999) (width 0.25) (layer F.Cu) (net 6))
 (segment (start 118.596839 68.884999) (end 118.031599 69.450239) (width 0.25) (layer F.Cu) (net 6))
 (segment (start 120.205601 68.319759) (end 119.640361 68.884999) (width 0.25) (layer F.Cu) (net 6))
 (segment (start 120.205601 64.370239) (end 120.205601 68.319759) (width 0.25) (layer F.Cu) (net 6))
 (segment (start 117.310361 61.474999) (end 120.205601 64.370239) (width 0.25) (layer F.Cu) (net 6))
 (segment (start 54.080788 61.474999) (end 117.310361 61.474999) (width 0.25) (layer F.Cu) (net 6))
 (segment (start 118.356601 76.830001) (end 119.1186 77.592) (width 0.25) (layer F.Cu) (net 6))
 (segment (start 119.640361 68.884999) (end 118.596839 68.884999) (width 0.25) (layer F.Cu) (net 6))
 (segment (start 53.96 61.595787) (end 54.080788 61.474999) (width 0.25) (layer F.Cu) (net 6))
 (segment (start 53.96 63.01) (end 53.96 61.595787) (width 0.25) (layer F.Cu) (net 6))
 (segment (start 107.871599 68.884999) (end 118.356601 79.370001) (width 0.25) (layer B.Cu) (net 10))
 (segment (start 103.484999 68.884999) (end 107.871599 68.884999) (width 0.25) (layer B.Cu) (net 10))
 (segment (start 118.356601 79.370001) (end 119.1186 80.132) (width 0.25) (layer B.Cu) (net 10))
 (segment (start 103.034999 68.434999) (end 103.484999 68.884999) (width 0.25) (layer B.Cu) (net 10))
 (segment (start 88.16 68.434999) (end 103.034999 68.434999) (width 0.25) (layer B.Cu) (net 10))
 (segment (start 82.525001 62.8) (end 88.16 68.434999) (width 0.25) (layer B.Cu) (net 10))
 (segment (start 77 62.8) (end 82.525001 62.8) (width 0.25) (layer B.Cu) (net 10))
 (segment (start 78.899999 72.285001) (end 72 65.385002) (width 0.25) (layer B.Cu) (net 9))
 (segment (start 99.360001 72.285001) (end 78.899999 72.285001) (width 0.25) (layer B.Cu) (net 9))
 (segment (start 100.220003 71.424999) (end 99.360001 72.285001) (width 0.25) (layer B.Cu) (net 9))
 (segment (start 107.871599 71.424999) (end 100.220003 71.424999) (width 0.25) (layer B.Cu) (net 9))
 (segment (start 72 64.214213) (end 72 62.8) (width 0.25) (layer B.Cu) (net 9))
 (segment (start 72 65.385002) (end 72 64.214213) (width 0.25) (layer B.Cu) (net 9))
 (segment (start 119.1186 82.672) (end 107.871599 71.424999) (width 0.25) (layer B.Cu) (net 9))
 (segment (start 118.356601 85.973999) (end 119.1186 85.212) (width 0.25) (layer F.Cu) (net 15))
 (segment (start 112.951599 91.379001) (end 118.356601 85.973999) (width 0.25) (layer F.Cu) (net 15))
 (segment (start 103.720999 91.379001) (end 112.951599 91.379001) (width 0.25) (layer F.Cu) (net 15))
 (segment (start 93.915999 94.415999) (end 100.784001 94.415999) (width 0.25) (layer F.Cu) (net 15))
 (segment (start 92.9 93.4) (end 93.915999 94.415999) (width 0.25) (layer F.Cu) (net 15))
 (segment (start 100.9 94.3) (end 103.720999 91.379001) (width 0.25) (layer F.Cu) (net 15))
 (segment (start 100.784001 94.415999) (end 100.9 94.3) (width 0.25) (layer F.Cu) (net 15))
 (segment (start 42.126009 89.813991) (end 100.227847 89.813991) (width 0.25) (layer B.Cu) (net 11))
 (segment (start 38.56 93.38) (end 42.126009 89.813991) (width 0.25) (layer B.Cu) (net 11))
 (segment (start 117.665601 89.204999) (end 118.356601 88.513999) (width 0.25) (layer B.Cu) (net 11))
 (segment (start 118.356601 88.513999) (end 119.1186 87.752) (width 0.25) (layer B.Cu) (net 11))
 (segment (start 100.836839 89.204999) (end 117.665601 89.204999) (width 0.25) (layer B.Cu) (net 11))
 (segment (start 100.227847 89.813991) (end 100.836839 89.204999) (width 0.25) (layer B.Cu) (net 11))
 (segment (start 118.356601 91.053999) (end 119.1186 90.292) (width 0.25) (layer F.Cu) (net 3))
 (segment (start 57.345328 99.15001) (end 110.26059 99.15001) (width 0.25) (layer F.Cu) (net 3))
 (segment (start 50.118999 91.923681) (end 57.345328 99.15001) (width 0.25) (layer F.Cu) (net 3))
 (segment (start 110.26059 99.15001) (end 118.356601 91.053999) (width 0.25) (layer F.Cu) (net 3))
 (segment (start 50.118999 88.504953) (end 50.118999 91.923681) (width 0.25) (layer F.Cu) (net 3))
 (segment (start 34.914999 73.300953) (end 50.118999 88.504953) (width 0.25) (layer F.Cu) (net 3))
 (segment (start 34.914999 64.025001) (end 34.914999 73.300953) (width 0.25) (layer F.Cu) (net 3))
 (segment (start 35.99 62.95) (end 34.914999 64.025001) (width 0.25) (layer F.Cu) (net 3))
 (segment (start 118.04097 92.832) (end 119.1186 92.832) (width 0.25) (layer B.Cu) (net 4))
 (segment (start 111.473997 98.475001) (end 117.116998 92.832) (width 0.25) (layer B.Cu) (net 4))
 (segment (start 38.670319 98.475001) (end 111.473997 98.475001) (width 0.25) (layer B.Cu) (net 4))
 (segment (start 31.564999 68.589999) (end 31.564999 91.369681) (width 0.25) (layer B.Cu) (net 4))
 (segment (start 34.876003 68.524999) (end 31.629999 68.524999) (width 0.25) (layer B.Cu) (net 4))
 (segment (start 40.451002 62.95) (end 34.876003 68.524999) (width 0.25) (layer B.Cu) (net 4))
 (segment (start 117.116998 92.832) (end 118.04097 92.832) (width 0.25) (layer B.Cu) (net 4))
 (segment (start 31.564999 91.369681) (end 38.670319 98.475001) (width 0.25) (layer B.Cu) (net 4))
 (segment (start 31.629999 68.524999) (end 31.564999 68.589999) (width 0.25) (layer B.Cu) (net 4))
 (segment (start 40.99 62.95) (end 40.451002 62.95) (width 0.25) (layer B.Cu) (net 4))
 (segment (start 103.136601 74.290001) (end 103.8986 75.052) (width 0.25) (layer F.Cu) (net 2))
 (segment (start 57.916319 72.938999) (end 101.785599 72.938999) (width 0.25) (layer F.Cu) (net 2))
 (segment (start 101.785599 72.938999) (end 103.136601 74.290001) (width 0.25) (layer F.Cu) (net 2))
 (segment (start 54.475318 76.38) (end 57.916319 72.938999) (width 0.25) (layer F.Cu) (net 2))
 (segment (start 42.06 76.38) (end 40.99 77.45) (width 0.25) (layer F.Cu) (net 2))
 (segment (start 43.14 76.38) (end 42.06 76.38) (width 0.25) (layer F.Cu) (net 2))
 (segment (start 43.14 76.38) (end 54.475318 76.38) (width 0.25) (layer F.Cu) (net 2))
 (segment (start 95 64.11) (end 95 62.86) (width 0.25) (layer B.Cu) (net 22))
 (segment (start 103.8986 64.892) (end 95.762 64.892) (width 0.25) (layer B.Cu) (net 22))
 (segment (start 95 64.13) (end 95 62.86) (width 0.25) (layer B.Cu) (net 22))
 (segment (start 95.762 64.892) (end 95 64.13) (width 0.25) (layer B.Cu) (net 22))
 (segment (start 94.572 67.432) (end 103.8986 67.432) (width 0.25) (layer B.Cu) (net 21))
 (segment (start 90 62.86) (end 94.572 67.432) (width 0.25) (layer B.Cu) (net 21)))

